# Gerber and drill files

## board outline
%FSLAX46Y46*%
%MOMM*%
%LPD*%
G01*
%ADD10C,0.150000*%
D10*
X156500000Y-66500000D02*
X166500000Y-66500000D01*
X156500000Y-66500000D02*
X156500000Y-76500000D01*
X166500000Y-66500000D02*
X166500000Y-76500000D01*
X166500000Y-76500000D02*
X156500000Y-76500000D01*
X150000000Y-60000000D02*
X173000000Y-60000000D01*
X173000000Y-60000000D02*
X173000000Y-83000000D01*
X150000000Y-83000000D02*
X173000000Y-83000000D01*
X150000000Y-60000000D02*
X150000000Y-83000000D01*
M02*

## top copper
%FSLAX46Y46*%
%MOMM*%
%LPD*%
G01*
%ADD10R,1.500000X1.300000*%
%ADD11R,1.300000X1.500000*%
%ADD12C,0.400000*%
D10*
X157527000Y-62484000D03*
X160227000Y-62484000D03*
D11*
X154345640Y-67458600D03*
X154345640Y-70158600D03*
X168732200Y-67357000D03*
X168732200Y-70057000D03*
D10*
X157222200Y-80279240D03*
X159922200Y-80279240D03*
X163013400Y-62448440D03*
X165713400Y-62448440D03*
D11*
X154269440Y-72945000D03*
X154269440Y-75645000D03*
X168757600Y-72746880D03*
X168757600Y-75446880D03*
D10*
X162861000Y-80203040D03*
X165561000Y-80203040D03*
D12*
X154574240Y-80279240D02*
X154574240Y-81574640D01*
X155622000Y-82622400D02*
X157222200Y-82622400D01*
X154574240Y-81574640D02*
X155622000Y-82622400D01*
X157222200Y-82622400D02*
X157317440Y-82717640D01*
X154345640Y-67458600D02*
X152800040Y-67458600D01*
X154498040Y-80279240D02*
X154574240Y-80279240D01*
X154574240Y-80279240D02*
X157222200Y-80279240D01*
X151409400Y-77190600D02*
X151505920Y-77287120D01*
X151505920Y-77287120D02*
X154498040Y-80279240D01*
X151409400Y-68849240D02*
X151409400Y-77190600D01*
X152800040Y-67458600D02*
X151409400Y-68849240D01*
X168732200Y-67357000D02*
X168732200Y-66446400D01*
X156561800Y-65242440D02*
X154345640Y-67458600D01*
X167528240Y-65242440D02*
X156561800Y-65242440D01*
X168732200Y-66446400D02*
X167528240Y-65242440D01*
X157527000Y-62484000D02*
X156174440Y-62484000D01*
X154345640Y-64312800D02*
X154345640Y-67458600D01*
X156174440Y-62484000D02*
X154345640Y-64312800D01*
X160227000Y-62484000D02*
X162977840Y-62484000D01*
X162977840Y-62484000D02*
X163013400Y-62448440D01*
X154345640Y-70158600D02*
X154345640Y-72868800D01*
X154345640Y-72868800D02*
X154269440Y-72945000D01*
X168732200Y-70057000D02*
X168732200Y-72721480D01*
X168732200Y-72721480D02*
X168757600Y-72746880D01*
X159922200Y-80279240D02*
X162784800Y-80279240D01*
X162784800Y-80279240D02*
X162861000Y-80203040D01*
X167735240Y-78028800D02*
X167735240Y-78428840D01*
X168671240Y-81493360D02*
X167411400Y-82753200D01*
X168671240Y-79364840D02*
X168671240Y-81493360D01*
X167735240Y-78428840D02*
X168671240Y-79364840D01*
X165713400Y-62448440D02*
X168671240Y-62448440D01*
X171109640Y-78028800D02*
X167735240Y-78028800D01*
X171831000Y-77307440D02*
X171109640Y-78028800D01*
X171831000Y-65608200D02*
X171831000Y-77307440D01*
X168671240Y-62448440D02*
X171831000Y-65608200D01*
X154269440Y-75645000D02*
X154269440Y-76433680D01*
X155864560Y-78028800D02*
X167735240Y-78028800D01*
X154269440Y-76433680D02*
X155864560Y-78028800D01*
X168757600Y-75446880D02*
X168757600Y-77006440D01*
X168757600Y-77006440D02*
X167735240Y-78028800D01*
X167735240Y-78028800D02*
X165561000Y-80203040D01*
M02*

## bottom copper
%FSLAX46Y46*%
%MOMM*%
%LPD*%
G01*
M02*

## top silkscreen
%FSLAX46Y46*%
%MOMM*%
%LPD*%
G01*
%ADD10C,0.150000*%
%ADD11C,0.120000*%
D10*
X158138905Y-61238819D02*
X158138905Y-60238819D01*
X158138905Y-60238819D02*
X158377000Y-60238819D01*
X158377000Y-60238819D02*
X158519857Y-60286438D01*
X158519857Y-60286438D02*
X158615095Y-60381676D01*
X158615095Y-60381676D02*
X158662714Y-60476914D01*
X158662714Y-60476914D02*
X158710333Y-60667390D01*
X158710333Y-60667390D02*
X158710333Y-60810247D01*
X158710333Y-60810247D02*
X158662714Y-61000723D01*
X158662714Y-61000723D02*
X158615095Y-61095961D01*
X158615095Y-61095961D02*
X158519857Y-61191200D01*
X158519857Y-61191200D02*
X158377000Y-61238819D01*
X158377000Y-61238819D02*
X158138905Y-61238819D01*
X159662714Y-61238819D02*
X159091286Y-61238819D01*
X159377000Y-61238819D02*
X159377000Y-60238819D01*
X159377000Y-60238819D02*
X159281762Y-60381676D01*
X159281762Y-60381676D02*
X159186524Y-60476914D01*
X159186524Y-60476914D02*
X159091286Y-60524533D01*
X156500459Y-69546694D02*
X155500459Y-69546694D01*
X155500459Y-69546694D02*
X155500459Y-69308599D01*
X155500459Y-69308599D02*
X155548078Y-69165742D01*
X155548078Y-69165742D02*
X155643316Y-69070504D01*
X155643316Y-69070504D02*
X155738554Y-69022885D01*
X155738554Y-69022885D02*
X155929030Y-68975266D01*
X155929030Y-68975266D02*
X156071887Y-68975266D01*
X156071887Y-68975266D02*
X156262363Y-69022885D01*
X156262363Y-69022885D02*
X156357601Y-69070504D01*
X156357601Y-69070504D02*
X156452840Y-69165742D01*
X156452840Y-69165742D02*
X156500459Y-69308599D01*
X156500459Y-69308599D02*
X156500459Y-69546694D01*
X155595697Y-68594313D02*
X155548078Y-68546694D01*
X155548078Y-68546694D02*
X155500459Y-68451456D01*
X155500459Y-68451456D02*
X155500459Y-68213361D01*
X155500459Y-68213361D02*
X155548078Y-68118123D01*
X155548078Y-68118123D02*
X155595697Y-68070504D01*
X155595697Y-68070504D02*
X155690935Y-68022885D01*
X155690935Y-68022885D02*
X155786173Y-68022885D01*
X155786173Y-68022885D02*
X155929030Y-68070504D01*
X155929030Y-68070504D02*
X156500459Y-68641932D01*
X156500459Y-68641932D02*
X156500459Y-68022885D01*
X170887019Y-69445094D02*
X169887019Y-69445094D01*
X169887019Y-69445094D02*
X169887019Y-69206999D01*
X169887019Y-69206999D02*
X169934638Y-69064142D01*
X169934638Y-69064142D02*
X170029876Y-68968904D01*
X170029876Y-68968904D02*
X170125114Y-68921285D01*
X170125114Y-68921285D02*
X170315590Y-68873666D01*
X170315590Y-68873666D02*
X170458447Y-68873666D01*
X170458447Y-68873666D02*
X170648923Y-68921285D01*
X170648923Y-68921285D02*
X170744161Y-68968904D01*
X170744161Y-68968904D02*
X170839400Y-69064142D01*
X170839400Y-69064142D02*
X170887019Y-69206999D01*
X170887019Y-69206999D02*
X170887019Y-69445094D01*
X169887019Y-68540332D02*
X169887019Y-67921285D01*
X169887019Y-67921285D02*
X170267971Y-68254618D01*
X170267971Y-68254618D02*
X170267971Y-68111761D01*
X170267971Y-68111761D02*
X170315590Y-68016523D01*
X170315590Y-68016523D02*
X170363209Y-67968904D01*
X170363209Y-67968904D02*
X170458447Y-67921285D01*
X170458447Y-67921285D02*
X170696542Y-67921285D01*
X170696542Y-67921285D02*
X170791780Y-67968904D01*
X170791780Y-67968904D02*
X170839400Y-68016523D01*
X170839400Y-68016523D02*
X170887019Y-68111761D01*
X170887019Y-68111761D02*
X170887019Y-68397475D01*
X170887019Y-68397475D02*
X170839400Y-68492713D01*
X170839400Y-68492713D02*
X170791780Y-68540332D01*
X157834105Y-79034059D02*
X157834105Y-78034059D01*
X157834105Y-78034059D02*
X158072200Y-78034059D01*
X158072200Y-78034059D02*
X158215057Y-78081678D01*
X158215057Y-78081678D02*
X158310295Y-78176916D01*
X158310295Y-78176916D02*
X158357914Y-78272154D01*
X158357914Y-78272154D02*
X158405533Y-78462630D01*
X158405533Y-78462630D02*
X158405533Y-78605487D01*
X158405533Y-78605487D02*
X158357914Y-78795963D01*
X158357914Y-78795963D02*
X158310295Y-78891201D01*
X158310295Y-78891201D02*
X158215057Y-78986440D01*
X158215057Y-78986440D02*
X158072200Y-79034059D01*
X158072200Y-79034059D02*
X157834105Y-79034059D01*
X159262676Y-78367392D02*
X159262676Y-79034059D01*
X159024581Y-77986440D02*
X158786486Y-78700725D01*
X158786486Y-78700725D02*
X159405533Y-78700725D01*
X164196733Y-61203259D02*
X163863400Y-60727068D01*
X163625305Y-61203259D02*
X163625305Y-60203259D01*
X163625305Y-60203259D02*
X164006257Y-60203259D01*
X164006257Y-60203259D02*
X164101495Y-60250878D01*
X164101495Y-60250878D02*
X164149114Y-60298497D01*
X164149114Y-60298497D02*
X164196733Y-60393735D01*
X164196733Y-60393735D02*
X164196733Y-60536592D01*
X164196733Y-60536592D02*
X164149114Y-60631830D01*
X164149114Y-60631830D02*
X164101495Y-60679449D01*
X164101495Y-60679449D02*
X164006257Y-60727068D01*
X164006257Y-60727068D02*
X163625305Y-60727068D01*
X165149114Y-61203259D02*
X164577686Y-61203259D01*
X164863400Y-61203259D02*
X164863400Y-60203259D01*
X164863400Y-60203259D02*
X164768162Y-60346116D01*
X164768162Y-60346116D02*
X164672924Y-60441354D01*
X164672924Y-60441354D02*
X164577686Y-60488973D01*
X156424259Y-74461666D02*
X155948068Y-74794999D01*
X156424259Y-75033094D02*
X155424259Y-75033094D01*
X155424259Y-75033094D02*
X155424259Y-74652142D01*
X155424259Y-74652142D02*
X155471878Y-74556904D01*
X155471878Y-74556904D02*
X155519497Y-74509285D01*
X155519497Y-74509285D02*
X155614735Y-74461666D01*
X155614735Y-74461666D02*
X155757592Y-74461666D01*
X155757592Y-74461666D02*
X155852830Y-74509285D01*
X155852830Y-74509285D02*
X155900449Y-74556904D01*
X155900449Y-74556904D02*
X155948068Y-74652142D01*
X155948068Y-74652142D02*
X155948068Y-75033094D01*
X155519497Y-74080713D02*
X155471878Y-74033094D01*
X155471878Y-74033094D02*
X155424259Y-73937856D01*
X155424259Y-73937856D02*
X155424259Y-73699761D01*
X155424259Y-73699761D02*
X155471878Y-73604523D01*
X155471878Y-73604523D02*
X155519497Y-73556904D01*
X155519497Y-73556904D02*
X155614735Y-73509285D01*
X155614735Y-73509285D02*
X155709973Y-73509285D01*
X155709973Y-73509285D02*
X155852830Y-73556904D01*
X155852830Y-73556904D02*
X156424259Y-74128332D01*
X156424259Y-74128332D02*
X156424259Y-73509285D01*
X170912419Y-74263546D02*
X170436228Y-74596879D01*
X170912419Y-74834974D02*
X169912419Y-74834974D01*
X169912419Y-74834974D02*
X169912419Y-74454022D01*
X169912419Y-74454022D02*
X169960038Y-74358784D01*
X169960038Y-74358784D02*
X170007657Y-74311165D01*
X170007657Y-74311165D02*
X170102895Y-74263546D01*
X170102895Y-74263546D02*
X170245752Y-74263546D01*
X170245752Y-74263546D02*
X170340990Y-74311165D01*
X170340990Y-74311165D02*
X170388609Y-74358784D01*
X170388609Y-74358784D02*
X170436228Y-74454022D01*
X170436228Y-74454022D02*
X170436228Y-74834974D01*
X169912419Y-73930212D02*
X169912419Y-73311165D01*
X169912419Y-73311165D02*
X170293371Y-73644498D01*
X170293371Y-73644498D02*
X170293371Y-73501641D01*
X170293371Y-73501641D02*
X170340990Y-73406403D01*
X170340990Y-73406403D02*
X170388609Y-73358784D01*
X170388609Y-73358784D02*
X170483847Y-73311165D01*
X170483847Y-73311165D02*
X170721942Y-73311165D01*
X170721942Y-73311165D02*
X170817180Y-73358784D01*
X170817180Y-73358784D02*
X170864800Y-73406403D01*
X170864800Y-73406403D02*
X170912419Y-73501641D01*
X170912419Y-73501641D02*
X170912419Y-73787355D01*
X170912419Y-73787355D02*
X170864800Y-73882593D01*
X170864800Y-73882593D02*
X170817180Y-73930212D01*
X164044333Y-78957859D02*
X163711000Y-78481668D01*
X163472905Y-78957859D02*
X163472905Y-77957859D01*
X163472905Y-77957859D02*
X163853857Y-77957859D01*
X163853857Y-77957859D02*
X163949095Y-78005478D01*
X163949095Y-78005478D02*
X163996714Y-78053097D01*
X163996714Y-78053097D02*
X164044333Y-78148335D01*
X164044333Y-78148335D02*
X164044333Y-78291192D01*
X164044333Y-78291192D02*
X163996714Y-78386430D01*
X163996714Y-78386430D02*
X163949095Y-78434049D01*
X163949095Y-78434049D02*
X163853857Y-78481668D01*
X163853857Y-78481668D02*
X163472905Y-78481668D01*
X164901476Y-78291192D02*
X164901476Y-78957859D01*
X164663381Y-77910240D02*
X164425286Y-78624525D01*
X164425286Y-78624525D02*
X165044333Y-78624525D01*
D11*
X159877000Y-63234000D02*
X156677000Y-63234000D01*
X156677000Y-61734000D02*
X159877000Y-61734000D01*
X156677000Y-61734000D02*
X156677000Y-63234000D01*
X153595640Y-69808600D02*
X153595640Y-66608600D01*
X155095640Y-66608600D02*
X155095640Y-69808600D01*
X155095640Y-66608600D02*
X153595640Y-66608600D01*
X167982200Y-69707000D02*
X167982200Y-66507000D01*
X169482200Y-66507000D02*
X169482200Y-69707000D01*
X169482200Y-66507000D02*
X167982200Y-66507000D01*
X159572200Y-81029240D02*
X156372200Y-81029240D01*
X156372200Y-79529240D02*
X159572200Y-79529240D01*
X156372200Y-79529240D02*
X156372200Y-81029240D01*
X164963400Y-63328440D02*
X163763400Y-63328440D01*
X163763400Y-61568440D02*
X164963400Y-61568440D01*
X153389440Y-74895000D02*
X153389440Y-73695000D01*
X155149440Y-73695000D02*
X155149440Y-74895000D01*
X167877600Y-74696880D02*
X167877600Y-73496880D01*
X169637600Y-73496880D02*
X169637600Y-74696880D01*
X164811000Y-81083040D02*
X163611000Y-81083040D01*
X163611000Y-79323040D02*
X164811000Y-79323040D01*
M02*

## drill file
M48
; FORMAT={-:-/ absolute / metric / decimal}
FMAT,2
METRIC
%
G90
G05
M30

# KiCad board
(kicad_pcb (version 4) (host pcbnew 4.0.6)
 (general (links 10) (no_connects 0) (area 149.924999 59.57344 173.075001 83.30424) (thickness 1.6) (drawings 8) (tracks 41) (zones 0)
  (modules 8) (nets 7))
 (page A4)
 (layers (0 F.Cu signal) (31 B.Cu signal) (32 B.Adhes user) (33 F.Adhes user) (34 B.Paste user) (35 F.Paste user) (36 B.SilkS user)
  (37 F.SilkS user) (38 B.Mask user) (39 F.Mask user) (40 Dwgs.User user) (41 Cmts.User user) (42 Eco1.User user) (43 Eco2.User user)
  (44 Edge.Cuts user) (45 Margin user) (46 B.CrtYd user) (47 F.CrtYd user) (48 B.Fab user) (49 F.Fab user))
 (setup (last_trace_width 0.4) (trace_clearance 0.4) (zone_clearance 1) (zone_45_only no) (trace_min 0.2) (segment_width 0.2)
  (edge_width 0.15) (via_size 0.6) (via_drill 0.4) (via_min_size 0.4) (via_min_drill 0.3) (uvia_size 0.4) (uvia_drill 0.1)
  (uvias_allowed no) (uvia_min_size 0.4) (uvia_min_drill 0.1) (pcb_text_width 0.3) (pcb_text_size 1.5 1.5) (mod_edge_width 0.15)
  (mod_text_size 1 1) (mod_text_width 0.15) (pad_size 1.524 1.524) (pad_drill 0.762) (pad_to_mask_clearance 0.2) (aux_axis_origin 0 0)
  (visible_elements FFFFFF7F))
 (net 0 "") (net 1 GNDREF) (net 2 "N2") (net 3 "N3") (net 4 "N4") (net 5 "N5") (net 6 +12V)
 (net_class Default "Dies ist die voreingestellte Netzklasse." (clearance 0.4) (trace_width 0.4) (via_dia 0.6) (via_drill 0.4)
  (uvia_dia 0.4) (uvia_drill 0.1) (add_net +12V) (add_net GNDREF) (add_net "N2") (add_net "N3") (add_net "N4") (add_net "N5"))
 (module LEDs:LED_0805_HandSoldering (layer F.Cu) (at 158.877 62.484)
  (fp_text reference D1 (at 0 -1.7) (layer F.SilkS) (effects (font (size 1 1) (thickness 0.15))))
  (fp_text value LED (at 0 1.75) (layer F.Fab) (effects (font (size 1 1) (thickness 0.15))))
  (fp_line (start 1 0.75) (end -2.2 0.75) (layer F.SilkS) (width 0.12))
  (fp_line (start -2.2 -0.75) (end 1 -0.75) (layer F.SilkS) (width 0.12))
  (fp_line (start -2.2 -0.75) (end -2.2 0.75) (layer F.SilkS) (width 0.12))
  (pad 1 smd rect (at -1.35 0) (size 1.5 1.3) (layers F.Cu F.Paste F.Mask) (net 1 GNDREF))
  (pad 2 smd rect (at 1.35 0) (size 1.5 1.3) (layers F.Cu F.Paste F.Mask) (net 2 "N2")))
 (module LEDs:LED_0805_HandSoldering (layer F.Cu) (at 154.34564 68.8086 270)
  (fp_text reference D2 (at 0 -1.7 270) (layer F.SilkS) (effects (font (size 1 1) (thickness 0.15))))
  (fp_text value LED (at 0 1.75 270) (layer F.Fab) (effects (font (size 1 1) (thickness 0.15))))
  (fp_line (start 1 0.75) (end -2.2 0.75) (layer F.SilkS) (width 0.12))
  (fp_line (start -2.2 -0.75) (end 1 -0.75) (layer F.SilkS) (width 0.12))
  (fp_line (start -2.2 -0.75) (end -2.2 0.75) (layer F.SilkS) (width 0.12))
  (pad 1 smd rect (at -1.35 0 270) (size 1.5 1.3) (layers F.Cu F.Paste F.Mask) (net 1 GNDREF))
  (pad 2 smd rect (at 1.35 0 270) (size 1.5 1.3) (layers F.Cu F.Paste F.Mask) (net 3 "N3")))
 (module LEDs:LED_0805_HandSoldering (layer F.Cu) (at 168.7322 68.707 270)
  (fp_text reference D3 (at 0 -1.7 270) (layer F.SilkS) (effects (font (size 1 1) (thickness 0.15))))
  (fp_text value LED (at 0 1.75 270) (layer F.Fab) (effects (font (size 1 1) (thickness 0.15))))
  (fp_line (start 1 0.75) (end -2.2 0.75) (layer F.SilkS) (width 0.12))
  (fp_line (start -2.2 -0.75) (end 1 -0.75) (layer F.SilkS) (width 0.12))
  (fp_line (start -2.2 -0.75) (end -2.2 0.75) (layer F.SilkS) (width 0.12))
  (pad 1 smd rect (at -1.35 0 270) (size 1.5 1.3) (layers F.Cu F.Paste F.Mask) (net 1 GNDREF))
  (pad 2 smd rect (at 1.35 0 270) (size 1.5 1.3) (layers F.Cu F.Paste F.Mask) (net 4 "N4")))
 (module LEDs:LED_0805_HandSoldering (layer F.Cu) (at 158.5722 80.27924)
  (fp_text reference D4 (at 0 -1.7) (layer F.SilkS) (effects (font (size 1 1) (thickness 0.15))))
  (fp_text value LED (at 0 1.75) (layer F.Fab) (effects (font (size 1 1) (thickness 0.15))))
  (fp_line (start 1 0.75) (end -2.2 0.75) (layer F.SilkS) (width 0.12))
  (fp_line (start -2.2 -0.75) (end 1 -0.75) (layer F.SilkS) (width 0.12))
  (fp_line (start -2.2 -0.75) (end -2.2 0.75) (layer F.SilkS) (width 0.12))
  (pad 1 smd rect (at -1.35 0) (size 1.5 1.3) (layers F.Cu F.Paste F.Mask) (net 1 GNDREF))
  (pad 2 smd rect (at 1.35 0) (size 1.5 1.3) (layers F.Cu F.Paste F.Mask) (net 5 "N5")))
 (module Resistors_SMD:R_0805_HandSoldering (layer F.Cu) (at 164.3634 62.44844)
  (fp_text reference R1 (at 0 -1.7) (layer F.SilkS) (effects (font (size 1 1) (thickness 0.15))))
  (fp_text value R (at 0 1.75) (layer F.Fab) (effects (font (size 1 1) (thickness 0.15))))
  (fp_line (start 0.6 0.88) (end -0.6 0.88) (layer F.SilkS) (width 0.12))
  (fp_line (start -0.6 -0.88) (end 0.6 -0.88) (layer F.SilkS) (width 0.12))
  (pad 1 smd rect (at -1.35 0) (size 1.5 1.3) (layers F.Cu F.Paste F.Mask) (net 2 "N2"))
  (pad 2 smd rect (at 1.35 0) (size 1.5 1.3) (layers F.Cu F.Paste F.Mask) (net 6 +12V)))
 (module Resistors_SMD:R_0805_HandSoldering (layer F.Cu) (at 154.26944 74.295 270)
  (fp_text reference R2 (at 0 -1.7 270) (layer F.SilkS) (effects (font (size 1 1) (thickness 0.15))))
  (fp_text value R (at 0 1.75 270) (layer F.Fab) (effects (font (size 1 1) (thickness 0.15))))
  (fp_line (start 0.6 0.88) (end -0.6 0.88) (layer F.SilkS) (width 0.12))
  (fp_line (start -0.6 -0.88) (end 0.6 -0.88) (layer F.SilkS) (width 0.12))
  (pad 1 smd rect (at -1.35 0 270) (size 1.5 1.3) (layers F.Cu F.Paste F.Mask) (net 3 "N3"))
  (pad 2 smd rect (at 1.35 0 270) (size 1.5 1.3) (layers F.Cu F.Paste F.Mask) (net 6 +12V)))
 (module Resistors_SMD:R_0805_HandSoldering (layer F.Cu) (at 168.7576 74.09688 270)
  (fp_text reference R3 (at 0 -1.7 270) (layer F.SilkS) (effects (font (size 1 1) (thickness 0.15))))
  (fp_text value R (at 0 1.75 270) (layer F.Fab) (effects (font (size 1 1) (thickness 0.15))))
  (fp_line (start 0.6 0.88) (end -0.6 0.88) (layer F.SilkS) (width 0.12))
  (fp_line (start -0.6 -0.88) (end 0.6 -0.88) (layer F.SilkS) (width 0.12))
  (pad 1 smd rect (at -1.35 0 270) (size 1.5 1.3) (layers F.Cu F.Paste F.Mask) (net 4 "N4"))
  (pad 2 smd rect (at 1.35 0 270) (size 1.5 1.3) (layers F.Cu F.Paste F.Mask) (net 6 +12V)))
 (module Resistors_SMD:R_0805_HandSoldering (layer F.Cu) (at 164.211 80.20304)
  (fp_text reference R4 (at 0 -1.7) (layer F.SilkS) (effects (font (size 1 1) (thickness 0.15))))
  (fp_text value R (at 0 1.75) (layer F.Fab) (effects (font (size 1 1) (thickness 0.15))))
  (fp_line (start 0.6 0.88) (end -0.6 0.88) (layer F.SilkS) (width 0.12))
  (fp_line (start -0.6 -0.88) (end 0.6 -0.88) (layer F.SilkS) (width 0.12))
  (pad 1 smd rect (at -1.35 0) (size 1.5 1.3) (layers F.Cu F.Paste F.Mask) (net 5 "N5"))
  (pad 2 smd rect (at 1.35 0) (size 1.5 1.3) (layers F.Cu F.Paste F.Mask) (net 6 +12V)))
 (gr_line (start 156.5 66.5) (end 166.5 66.5) (angle 90) (layer Edge.Cuts) (width 0.15))
 (gr_line (start 156.5 66.5) (end 156.5 76.5) (angle 90) (layer Edge.Cuts) (width 0.15))
 (gr_line (start 166.5 66.5) (end 166.5 76.5) (angle 90) (layer Edge.Cuts) (width 0.15))
 (gr_line (start 166.5 76.5) (end 156.5 76.5) (angle 90) (layer Edge.Cuts) (width 0.15))
 (gr_line (start 150 60) (end 173 60) (angle 90) (layer Edge.Cuts) (width 0.15))
 (gr_line (start 173 60) (end 173 83) (angle 90) (layer Edge.Cuts) (width 0.15))
 (gr_line (start 150 83) (end 173 83) (angle 90) (layer Edge.Cuts) (width 0.15))
 (gr_line (start 150 60) (end 150 83) (angle 90) (layer Edge.Cuts) (width 0.15))
 (segment (start 154.57424 80.27924) (end 154.57424 81.57464) (width 0.4) (layer F.Cu) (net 1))
 (segment (start 155.622 82.6224) (end 157.2222 82.6224) (width 0.4) (layer F.Cu) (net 1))
 (segment (start 154.57424 81.57464) (end 155.622 82.6224) (width 0.4) (layer F.Cu) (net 1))
 (segment (start 157.2222 82.6224) (end 157.31744 82.71764) (width 0.4) (layer F.Cu) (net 1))
 (segment (start 154.34564 67.4586) (end 152.80004 67.4586) (width 0.4) (layer F.Cu) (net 1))
 (segment (start 154.49804 80.27924) (end 154.57424 80.27924) (width 0.4) (layer F.Cu) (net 1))
 (segment (start 154.57424 80.27924) (end 157.2222 80.27924) (width 0.4) (layer F.Cu) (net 1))
 (segment (start 151.4094 77.1906) (end 151.50592 77.28712) (width 0.4) (layer F.Cu) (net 1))
 (segment (start 151.50592 77.28712) (end 154.49804 80.27924) (width 0.4) (layer F.Cu) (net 1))
 (segment (start 151.4094 68.84924) (end 151.4094 77.1906) (width 0.4) (layer F.Cu) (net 1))
 (segment (start 152.80004 67.4586) (end 151.4094 68.84924) (width 0.4) (layer F.Cu) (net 1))
 (segment (start 168.7322 67.357) (end 168.7322 66.4464) (width 0.4) (layer F.Cu) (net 1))
 (segment (start 156.5618 65.24244) (end 154.34564 67.4586) (width 0.4) (layer F.Cu) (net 1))
 (segment (start 167.52824 65.24244) (end 156.5618 65.24244) (width 0.4) (layer F.Cu) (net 1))
 (segment (start 168.7322 66.4464) (end 167.52824 65.24244) (width 0.4) (layer F.Cu) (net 1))
 (segment (start 157.527 62.484) (end 156.17444 62.484) (width 0.4) (layer F.Cu) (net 1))
 (segment (start 154.34564 64.3128) (end 154.34564 67.4586) (width 0.4) (layer F.Cu) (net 1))
 (segment (start 156.17444 62.484) (end 154.34564 64.3128) (width 0.4) (layer F.Cu) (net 1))
 (segment (start 160.227 62.484) (end 162.97784 62.484) (width 0.4) (layer F.Cu) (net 2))
 (segment (start 162.97784 62.484) (end 163.0134 62.44844) (width 0.4) (layer F.Cu) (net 2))
 (segment (start 154.34564 70.1586) (end 154.34564 72.8688) (width 0.4) (layer F.Cu) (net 3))
 (segment (start 154.34564 72.8688) (end 154.26944 72.945) (width 0.4) (layer F.Cu) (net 3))
 (segment (start 168.7322 70.057) (end 168.7322 72.72148) (width 0.4) (layer F.Cu) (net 4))
 (segment (start 168.7322 72.72148) (end 168.7576 72.74688) (width 0.4) (layer F.Cu) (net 4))
 (segment (start 159.9222 80.27924) (end 162.7848 80.27924) (width 0.4) (layer F.Cu) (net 5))
 (segment (start 162.7848 80.27924) (end 162.861 80.20304) (width 0.4) (layer F.Cu) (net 5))
 (segment (start 167.73524 78.0288) (end 167.73524 78.42884) (width 0.4) (layer F.Cu) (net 6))
 (segment (start 168.67124 81.49336) (end 167.4114 82.7532) (width 0.4) (layer F.Cu) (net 6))
 (segment (start 168.67124 79.36484) (end 168.67124 81.49336) (width 0.4) (layer F.Cu) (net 6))
 (segment (start 167.73524 78.42884) (end 168.67124 79.36484) (width 0.4) (layer F.Cu) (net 6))
 (segment (start 165.7134 62.44844) (end 168.67124 62.44844) (width 0.4) (layer F.Cu) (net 6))
 (segment (start 171.10964 78.0288) (end 167.73524 78.0288) (width 0.4) (layer F.Cu) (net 6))
 (segment (start 171.831 77.30744) (end 171.10964 78.0288) (width 0.4) (layer F.Cu) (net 6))
 (segment (start 171.831 65.6082) (end 171.831 77.30744) (width 0.4) (layer F.Cu) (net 6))
 (segment (start 168.67124 62.44844) (end 171.831 65.6082) (width 0.4) (layer F.Cu) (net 6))
 (segment (start 154.26944 75.645) (end 154.26944 76.43368) (width 0.4) (layer F.Cu) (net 6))
 (segment (start 155.86456 78.0288) (end 167.73524 78.0288) (width 0.4) (layer F.Cu) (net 6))
 (segment (start 154.26944 76.43368) (end 155.86456 78.0288) (width 0.4) (layer F.Cu) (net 6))
 (segment (start 168.7576 75.44688) (end 168.7576 77.00644) (width 0.4) (layer F.Cu) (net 6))
 (segment (start 168.7576 77.00644) (end 167.73524 78.0288) (width 0.4) (layer F.Cu) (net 6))
 (segment (start 167.73524 78.0288) (end 165.561 80.20304) (width 0.4) (layer F.Cu) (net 6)))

